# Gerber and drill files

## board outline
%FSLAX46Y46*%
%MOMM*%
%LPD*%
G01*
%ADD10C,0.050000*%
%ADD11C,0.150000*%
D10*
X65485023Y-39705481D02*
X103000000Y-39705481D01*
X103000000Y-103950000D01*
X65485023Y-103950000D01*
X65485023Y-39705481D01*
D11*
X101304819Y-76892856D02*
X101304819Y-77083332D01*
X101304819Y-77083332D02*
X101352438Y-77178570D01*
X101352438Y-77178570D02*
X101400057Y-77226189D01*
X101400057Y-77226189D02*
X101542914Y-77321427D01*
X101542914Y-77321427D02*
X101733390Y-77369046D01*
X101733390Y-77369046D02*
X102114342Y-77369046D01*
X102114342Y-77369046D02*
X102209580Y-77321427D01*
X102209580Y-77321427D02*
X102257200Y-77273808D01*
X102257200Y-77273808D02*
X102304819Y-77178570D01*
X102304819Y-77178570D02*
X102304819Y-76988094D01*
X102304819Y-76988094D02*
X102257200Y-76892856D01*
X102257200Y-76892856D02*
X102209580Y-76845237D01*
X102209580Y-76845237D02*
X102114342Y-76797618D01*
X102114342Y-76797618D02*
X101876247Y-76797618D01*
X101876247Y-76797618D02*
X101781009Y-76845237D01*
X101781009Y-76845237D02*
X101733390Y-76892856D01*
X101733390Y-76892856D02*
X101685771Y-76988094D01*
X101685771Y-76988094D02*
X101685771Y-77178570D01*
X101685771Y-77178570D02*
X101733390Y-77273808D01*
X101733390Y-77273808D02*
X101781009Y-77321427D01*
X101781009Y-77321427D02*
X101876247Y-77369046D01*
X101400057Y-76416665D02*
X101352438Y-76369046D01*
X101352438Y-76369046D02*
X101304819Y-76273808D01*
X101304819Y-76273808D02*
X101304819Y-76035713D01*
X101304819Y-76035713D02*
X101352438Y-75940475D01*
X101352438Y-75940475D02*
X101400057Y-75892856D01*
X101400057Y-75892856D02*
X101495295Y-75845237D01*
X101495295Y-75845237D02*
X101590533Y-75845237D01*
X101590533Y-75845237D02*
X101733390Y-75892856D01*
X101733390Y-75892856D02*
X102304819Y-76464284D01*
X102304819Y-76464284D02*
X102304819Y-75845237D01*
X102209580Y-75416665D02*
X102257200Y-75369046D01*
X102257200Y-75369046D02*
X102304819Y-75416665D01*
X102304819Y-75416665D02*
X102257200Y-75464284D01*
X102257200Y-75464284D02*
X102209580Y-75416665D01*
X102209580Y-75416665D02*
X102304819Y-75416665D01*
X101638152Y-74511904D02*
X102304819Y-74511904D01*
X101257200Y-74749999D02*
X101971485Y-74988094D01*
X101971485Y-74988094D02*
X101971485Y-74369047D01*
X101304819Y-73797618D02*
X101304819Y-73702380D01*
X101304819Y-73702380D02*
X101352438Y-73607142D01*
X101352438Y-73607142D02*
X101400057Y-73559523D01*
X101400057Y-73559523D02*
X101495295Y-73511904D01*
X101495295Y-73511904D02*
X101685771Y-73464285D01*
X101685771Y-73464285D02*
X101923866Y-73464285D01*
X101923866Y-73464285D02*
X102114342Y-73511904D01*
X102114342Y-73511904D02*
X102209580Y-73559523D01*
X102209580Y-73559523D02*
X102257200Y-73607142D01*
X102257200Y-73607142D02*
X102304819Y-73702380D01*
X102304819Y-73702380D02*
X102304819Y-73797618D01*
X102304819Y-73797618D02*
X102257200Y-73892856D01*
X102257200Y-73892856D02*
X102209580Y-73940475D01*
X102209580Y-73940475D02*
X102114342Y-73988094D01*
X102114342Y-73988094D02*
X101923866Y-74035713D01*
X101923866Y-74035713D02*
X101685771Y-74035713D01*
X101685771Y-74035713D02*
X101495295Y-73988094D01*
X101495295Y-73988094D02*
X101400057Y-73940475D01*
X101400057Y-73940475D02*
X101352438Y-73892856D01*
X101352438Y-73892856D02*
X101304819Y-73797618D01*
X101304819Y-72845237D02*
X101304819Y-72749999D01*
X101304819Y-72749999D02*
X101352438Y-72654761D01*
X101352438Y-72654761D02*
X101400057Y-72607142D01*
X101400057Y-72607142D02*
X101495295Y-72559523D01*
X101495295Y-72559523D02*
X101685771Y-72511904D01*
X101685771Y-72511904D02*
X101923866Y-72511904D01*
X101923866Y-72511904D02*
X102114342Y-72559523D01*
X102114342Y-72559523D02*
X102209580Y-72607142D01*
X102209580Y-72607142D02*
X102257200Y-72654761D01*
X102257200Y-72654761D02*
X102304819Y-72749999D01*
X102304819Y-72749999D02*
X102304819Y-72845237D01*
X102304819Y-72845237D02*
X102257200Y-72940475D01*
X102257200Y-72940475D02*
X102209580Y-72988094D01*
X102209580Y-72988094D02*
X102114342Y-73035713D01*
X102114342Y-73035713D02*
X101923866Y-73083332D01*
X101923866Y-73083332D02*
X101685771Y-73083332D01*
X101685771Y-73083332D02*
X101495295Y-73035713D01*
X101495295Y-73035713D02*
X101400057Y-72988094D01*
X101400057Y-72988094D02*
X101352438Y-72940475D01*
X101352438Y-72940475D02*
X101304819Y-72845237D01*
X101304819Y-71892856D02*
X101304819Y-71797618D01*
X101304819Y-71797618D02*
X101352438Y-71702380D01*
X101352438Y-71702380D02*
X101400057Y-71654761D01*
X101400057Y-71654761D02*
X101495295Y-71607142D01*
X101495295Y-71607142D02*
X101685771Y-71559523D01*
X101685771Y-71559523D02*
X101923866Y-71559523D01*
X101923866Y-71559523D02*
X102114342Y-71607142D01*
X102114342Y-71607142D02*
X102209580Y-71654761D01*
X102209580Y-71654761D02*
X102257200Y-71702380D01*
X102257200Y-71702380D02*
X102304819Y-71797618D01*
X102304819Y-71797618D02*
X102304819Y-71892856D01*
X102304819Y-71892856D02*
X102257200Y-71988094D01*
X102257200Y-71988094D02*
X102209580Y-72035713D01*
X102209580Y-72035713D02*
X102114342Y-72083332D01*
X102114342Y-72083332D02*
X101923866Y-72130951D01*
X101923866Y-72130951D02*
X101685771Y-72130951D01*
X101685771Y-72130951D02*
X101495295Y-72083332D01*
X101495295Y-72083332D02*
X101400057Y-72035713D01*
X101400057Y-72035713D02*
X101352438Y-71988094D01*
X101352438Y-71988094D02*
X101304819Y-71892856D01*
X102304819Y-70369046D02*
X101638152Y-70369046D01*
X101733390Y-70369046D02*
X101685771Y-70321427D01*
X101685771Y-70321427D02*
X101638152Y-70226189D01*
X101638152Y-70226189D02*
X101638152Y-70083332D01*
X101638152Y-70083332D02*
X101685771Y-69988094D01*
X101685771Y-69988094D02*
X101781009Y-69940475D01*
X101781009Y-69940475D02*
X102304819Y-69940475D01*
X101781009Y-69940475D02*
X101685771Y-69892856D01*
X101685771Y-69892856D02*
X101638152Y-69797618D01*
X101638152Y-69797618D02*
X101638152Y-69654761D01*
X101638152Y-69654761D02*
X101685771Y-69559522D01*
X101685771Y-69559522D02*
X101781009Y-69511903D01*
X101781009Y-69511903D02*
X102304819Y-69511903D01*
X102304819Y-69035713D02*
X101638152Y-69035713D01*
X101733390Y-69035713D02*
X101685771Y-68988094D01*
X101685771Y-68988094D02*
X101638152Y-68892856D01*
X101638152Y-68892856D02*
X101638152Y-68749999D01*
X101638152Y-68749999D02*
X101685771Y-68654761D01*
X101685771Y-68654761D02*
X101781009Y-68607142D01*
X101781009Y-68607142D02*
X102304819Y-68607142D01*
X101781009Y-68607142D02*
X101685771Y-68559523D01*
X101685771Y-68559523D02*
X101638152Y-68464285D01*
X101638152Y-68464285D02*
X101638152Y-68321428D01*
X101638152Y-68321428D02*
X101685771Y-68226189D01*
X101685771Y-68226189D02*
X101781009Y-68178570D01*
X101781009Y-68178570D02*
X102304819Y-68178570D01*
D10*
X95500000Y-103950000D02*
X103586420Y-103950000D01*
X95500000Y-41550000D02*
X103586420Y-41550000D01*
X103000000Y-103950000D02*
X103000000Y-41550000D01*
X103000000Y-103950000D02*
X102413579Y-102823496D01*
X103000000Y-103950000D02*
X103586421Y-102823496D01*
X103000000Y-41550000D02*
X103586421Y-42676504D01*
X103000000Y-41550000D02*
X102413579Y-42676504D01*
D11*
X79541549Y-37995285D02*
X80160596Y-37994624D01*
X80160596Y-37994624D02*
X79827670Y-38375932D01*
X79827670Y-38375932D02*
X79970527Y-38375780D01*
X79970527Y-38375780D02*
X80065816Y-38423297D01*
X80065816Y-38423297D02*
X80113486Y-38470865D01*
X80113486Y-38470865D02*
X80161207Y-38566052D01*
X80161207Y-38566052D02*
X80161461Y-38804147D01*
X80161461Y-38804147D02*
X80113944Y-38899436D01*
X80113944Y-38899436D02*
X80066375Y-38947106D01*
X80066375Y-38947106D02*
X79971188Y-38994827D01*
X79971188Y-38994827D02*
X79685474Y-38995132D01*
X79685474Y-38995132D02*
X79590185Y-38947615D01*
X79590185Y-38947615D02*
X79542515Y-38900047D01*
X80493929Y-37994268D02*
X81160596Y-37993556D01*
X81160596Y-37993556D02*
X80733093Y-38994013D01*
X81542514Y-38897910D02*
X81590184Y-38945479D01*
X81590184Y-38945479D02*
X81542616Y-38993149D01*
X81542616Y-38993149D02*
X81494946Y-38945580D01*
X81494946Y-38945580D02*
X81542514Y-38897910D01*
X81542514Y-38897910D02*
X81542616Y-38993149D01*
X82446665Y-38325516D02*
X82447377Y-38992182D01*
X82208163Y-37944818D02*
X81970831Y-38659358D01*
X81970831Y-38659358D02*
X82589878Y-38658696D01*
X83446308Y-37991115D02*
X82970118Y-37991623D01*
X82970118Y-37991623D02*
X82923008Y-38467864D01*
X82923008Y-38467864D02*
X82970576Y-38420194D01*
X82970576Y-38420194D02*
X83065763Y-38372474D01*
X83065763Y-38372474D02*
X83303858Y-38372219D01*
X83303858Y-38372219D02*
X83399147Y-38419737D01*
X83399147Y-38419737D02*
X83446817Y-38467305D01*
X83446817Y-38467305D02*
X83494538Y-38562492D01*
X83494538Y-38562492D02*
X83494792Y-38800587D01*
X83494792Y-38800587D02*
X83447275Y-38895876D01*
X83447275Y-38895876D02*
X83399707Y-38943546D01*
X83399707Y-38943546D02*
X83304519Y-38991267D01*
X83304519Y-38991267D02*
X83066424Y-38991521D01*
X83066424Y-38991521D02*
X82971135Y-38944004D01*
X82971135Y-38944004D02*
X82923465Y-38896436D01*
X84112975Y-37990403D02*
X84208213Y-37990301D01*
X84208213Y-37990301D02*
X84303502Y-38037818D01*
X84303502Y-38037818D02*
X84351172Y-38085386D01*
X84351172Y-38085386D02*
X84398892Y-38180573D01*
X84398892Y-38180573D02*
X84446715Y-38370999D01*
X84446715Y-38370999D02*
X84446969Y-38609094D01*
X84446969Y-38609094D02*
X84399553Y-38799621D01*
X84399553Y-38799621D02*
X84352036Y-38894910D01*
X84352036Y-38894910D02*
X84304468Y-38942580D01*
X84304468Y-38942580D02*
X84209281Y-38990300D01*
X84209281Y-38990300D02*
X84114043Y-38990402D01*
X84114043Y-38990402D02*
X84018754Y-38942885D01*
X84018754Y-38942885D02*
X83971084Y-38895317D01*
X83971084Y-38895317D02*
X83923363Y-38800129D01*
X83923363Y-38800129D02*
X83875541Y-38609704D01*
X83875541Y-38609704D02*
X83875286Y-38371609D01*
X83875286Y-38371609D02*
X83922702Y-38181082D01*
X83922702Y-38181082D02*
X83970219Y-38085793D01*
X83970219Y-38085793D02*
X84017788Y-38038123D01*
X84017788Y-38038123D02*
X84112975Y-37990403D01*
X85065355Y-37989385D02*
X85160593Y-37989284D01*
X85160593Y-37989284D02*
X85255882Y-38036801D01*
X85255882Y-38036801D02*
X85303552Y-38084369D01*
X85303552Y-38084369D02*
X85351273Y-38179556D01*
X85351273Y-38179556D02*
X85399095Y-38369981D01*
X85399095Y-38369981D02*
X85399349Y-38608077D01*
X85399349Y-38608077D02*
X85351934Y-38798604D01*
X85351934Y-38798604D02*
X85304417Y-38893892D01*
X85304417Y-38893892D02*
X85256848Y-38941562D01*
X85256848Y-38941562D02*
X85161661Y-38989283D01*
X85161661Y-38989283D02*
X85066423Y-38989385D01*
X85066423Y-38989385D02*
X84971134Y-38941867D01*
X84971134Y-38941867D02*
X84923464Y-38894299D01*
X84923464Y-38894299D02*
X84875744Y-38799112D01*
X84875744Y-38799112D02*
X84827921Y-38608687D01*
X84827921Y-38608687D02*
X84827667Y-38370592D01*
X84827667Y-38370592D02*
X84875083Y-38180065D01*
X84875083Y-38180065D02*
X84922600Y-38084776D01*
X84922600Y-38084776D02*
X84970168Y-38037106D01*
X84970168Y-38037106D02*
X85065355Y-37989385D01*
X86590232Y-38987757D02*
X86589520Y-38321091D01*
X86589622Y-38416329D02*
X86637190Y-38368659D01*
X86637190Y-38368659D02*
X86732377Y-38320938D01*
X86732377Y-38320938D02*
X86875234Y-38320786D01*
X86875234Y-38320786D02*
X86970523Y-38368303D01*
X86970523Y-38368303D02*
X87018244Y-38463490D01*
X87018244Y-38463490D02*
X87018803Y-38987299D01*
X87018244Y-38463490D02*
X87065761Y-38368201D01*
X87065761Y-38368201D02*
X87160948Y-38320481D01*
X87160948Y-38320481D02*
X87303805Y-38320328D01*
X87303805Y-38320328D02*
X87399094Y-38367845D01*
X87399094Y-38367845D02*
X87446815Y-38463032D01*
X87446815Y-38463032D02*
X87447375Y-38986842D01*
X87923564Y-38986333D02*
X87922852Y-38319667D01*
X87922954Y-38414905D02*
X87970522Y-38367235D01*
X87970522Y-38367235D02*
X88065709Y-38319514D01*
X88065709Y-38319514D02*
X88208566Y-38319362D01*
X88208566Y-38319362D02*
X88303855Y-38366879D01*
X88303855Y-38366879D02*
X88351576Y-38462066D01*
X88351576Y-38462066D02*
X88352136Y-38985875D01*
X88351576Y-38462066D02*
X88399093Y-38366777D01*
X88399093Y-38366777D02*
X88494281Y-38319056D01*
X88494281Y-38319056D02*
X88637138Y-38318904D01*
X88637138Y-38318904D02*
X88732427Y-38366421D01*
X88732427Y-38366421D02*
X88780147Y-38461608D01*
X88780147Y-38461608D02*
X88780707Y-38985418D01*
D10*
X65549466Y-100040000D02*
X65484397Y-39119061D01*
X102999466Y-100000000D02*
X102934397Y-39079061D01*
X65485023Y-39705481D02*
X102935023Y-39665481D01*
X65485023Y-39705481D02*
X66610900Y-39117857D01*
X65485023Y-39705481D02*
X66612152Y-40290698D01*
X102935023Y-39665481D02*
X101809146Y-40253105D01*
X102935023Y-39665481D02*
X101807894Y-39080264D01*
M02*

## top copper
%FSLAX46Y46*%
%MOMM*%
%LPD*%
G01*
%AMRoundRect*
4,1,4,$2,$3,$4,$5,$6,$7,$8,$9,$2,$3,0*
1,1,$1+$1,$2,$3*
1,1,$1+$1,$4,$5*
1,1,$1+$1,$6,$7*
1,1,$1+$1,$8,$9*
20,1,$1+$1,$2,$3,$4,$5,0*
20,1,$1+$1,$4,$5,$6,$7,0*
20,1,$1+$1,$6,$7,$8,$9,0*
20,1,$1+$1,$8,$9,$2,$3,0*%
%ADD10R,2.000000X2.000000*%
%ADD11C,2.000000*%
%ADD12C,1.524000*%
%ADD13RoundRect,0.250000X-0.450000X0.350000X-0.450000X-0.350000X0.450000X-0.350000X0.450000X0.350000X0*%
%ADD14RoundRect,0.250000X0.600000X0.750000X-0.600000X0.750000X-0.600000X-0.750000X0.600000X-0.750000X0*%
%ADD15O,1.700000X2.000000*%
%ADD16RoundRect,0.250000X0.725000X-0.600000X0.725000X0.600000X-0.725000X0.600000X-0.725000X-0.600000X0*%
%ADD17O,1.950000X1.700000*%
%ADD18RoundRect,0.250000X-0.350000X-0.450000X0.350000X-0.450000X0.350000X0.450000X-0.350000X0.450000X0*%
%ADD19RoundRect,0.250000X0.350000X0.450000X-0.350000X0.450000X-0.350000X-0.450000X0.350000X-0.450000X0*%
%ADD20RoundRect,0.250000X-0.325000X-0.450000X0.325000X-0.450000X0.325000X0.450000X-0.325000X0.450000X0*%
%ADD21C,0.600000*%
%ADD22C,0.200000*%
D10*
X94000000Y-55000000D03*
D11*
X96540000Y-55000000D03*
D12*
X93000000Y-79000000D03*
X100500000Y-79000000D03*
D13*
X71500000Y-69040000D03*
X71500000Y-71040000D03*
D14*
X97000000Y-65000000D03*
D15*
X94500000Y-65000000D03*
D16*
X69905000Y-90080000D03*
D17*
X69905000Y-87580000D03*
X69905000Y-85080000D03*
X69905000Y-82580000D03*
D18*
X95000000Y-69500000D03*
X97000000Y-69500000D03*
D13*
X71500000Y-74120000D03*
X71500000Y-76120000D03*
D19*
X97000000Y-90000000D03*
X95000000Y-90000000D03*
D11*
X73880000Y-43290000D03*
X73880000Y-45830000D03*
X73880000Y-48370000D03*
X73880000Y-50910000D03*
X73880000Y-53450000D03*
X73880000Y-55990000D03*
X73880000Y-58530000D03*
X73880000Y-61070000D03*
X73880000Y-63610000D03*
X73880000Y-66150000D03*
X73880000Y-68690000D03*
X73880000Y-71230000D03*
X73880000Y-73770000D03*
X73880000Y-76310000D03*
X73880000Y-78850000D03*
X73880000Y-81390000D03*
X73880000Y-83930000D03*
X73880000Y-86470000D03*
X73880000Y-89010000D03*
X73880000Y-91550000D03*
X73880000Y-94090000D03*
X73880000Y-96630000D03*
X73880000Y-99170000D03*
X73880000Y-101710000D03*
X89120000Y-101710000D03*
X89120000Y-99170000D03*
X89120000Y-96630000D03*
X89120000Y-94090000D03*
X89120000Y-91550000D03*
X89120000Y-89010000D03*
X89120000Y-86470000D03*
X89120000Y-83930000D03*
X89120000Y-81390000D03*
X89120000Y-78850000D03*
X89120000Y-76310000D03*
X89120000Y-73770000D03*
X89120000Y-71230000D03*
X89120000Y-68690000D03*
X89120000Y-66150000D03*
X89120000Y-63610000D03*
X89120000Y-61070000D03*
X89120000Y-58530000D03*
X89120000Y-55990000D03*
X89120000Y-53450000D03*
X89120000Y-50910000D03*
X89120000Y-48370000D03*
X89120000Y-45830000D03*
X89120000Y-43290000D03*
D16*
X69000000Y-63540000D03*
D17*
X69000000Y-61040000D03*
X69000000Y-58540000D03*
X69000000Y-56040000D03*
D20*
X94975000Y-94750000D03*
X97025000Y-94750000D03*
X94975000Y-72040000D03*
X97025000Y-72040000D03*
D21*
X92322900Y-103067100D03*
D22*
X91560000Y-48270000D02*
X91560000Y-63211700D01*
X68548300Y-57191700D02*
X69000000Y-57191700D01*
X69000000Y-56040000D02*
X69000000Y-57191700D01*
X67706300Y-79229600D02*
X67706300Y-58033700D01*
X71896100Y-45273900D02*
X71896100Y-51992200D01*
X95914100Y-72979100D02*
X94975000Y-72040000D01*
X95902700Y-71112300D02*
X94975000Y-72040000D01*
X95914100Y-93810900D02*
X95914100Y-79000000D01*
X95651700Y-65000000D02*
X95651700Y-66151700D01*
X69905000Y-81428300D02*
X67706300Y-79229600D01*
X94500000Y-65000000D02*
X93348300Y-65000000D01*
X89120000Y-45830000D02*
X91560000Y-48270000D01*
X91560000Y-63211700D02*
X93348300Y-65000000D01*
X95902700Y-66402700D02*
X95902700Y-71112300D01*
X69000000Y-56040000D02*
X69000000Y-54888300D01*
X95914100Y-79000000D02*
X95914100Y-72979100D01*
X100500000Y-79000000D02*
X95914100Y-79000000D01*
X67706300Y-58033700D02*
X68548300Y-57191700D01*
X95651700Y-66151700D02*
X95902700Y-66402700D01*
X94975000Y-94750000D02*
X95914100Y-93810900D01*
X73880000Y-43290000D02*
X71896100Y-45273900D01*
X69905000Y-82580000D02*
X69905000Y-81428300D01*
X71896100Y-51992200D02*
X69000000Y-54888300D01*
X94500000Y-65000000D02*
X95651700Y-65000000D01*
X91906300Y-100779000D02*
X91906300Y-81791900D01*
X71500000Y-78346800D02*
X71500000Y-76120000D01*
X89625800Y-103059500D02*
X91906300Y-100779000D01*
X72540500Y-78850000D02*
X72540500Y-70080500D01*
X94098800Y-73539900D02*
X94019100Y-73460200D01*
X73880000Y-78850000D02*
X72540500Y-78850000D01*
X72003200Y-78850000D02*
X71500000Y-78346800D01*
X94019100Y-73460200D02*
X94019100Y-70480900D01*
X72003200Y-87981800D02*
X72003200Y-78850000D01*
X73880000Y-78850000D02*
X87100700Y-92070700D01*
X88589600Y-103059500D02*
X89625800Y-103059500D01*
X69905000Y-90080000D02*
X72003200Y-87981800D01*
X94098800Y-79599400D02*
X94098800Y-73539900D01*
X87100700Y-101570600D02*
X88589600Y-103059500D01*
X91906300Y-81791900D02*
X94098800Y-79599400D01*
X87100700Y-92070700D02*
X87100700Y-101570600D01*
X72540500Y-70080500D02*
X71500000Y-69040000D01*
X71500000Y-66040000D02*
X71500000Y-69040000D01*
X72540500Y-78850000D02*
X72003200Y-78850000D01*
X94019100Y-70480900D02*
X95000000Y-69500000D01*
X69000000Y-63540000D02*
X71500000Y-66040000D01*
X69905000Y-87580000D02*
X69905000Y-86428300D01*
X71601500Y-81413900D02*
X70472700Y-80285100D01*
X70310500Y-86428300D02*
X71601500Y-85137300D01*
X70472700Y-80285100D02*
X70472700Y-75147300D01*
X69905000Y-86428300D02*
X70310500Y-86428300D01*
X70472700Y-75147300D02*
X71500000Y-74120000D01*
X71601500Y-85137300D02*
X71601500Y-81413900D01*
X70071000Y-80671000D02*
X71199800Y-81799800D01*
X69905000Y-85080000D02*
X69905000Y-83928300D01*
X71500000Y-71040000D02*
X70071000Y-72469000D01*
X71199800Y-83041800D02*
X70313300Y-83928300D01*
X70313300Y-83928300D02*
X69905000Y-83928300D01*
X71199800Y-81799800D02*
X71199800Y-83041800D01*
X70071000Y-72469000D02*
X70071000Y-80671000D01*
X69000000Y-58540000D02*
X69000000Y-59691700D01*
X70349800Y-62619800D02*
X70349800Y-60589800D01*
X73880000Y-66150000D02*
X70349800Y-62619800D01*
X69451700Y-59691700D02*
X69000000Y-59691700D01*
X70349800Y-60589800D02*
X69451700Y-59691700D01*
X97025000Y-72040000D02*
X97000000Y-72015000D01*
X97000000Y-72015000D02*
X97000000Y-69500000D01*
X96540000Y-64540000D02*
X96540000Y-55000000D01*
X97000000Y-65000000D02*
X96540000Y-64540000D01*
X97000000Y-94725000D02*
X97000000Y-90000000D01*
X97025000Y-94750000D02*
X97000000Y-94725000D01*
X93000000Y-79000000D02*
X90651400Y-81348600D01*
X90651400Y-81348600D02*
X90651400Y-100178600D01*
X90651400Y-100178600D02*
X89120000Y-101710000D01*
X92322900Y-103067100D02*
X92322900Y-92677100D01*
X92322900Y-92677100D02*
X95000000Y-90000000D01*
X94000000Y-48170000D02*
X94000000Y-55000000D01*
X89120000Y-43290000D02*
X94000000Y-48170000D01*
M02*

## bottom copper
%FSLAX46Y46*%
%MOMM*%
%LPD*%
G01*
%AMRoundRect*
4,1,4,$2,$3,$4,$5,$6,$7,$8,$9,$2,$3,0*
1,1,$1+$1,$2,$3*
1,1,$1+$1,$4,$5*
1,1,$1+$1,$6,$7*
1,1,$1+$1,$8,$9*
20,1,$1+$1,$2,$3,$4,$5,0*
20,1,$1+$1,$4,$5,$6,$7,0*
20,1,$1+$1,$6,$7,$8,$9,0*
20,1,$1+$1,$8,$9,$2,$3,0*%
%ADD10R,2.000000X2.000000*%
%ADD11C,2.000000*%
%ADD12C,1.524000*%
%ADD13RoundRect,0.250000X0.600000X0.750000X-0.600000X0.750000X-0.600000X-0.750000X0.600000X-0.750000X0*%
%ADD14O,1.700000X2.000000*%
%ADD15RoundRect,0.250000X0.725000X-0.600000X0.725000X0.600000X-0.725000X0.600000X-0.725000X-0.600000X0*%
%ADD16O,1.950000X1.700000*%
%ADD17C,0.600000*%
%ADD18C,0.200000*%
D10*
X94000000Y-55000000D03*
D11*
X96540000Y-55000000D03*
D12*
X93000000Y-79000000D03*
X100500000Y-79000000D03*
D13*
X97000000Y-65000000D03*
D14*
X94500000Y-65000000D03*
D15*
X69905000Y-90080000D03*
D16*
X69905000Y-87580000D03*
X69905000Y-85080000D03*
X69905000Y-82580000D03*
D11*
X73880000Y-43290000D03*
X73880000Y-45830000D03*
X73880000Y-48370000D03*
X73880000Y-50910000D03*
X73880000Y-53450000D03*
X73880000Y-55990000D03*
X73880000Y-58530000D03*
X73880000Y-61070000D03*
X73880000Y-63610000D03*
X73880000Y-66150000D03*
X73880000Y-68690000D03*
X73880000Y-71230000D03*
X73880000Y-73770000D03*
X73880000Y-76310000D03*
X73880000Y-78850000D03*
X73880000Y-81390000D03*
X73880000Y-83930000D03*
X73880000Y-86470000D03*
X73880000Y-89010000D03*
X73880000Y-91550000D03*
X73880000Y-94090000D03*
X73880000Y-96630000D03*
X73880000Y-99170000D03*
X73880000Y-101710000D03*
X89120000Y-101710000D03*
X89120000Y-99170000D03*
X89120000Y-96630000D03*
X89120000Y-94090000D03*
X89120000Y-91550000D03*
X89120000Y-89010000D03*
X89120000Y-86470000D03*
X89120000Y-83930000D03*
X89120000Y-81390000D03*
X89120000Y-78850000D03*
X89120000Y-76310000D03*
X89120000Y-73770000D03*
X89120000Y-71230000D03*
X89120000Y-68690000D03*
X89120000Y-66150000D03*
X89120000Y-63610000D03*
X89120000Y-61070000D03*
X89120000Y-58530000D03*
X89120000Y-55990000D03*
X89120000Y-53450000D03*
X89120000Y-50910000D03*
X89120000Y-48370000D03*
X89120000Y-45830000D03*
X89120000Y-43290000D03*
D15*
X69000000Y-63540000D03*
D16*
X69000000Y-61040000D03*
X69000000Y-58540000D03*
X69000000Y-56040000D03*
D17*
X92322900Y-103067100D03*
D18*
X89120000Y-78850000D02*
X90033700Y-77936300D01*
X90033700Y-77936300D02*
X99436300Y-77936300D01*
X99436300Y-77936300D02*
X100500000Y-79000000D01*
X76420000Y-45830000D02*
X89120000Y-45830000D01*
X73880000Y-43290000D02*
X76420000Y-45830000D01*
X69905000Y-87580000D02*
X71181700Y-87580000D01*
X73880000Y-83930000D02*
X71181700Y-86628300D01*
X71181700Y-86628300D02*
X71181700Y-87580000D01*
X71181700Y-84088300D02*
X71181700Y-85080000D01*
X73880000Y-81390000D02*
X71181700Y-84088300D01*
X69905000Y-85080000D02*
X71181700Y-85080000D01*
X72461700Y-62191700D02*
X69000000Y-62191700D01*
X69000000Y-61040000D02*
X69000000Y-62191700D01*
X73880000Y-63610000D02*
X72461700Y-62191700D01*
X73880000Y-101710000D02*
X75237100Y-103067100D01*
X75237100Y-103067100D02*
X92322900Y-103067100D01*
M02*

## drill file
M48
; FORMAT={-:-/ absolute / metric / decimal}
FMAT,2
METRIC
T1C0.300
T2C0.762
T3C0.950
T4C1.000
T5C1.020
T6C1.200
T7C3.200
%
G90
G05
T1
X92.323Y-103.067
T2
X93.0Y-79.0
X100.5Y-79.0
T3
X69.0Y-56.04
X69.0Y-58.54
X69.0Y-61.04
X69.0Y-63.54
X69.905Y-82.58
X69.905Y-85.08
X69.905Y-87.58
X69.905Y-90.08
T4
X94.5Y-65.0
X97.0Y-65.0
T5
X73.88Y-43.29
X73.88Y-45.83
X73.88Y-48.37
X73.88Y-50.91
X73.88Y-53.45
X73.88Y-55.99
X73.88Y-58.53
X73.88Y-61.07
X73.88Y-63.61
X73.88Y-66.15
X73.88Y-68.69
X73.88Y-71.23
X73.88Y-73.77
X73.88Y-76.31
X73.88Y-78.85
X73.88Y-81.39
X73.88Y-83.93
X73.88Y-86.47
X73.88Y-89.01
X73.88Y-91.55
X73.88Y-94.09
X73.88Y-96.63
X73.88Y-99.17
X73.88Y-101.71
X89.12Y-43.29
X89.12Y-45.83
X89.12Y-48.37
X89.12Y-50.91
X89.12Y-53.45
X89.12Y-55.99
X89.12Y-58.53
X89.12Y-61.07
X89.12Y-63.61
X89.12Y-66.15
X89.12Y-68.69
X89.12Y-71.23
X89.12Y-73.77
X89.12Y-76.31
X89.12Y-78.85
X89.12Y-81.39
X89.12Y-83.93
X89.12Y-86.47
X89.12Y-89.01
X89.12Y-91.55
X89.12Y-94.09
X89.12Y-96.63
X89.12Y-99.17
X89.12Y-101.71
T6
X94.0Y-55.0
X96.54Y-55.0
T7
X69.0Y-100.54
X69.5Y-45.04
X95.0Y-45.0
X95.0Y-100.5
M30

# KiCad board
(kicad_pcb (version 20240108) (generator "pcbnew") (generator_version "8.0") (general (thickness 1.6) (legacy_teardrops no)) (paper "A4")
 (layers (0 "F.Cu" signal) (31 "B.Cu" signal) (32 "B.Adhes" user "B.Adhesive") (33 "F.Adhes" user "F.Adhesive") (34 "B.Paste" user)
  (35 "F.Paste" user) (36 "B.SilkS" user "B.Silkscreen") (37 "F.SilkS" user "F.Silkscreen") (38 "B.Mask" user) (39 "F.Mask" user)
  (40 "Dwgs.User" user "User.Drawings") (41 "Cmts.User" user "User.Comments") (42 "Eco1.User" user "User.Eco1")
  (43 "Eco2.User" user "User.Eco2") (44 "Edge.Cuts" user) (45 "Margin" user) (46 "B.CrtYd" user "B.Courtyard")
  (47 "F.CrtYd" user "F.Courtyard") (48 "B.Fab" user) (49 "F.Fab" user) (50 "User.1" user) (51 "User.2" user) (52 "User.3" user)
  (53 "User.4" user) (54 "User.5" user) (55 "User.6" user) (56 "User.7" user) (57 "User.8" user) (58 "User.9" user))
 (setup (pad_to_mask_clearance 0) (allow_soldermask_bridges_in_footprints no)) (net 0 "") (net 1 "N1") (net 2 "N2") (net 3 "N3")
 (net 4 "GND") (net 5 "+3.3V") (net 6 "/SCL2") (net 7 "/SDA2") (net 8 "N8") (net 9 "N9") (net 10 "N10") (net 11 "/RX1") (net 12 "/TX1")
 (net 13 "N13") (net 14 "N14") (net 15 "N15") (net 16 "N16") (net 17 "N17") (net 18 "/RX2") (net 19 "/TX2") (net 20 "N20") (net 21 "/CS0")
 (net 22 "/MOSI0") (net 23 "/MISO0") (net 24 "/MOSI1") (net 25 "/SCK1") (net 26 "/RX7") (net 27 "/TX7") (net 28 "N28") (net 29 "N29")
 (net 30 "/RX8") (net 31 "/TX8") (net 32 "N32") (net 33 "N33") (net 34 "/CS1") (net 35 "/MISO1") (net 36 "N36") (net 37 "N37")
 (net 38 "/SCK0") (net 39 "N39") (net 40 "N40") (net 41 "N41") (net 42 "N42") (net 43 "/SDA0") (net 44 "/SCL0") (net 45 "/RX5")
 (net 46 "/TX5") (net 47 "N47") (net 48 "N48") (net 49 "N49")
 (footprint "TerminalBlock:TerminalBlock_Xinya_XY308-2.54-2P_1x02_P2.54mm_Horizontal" (layer "F.Cu") (at 94 55)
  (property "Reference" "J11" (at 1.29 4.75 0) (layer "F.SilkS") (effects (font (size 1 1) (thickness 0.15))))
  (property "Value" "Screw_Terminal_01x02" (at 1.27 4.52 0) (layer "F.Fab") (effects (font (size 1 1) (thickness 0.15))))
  (pad "1" thru_hole rect (at 0 0) (size 2 2) (drill 1.2) (layers "*.Cu" "*.Mask") (remove_unused_layers no) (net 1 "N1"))
  (pad "2" thru_hole circle (at 2.54 0) (size 2 2) (drill 1.2) (layers "*.Cu" "*.Mask") (remove_unused_layers no) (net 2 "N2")))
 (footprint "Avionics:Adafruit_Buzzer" (layer "F.Cu") (at 97 79)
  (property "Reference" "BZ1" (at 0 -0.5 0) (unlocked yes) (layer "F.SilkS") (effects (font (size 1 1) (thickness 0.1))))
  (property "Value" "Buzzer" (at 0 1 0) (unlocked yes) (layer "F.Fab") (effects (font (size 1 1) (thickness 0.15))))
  (pad "1" thru_hole circle (at -4 0) (size 1.524 1.524) (drill 0.762) (layers "*.Cu" "*.Mask") (remove_unused_layers no) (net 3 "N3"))
  (pad "2" thru_hole circle (at 3.5 0) (size 1.524 1.524) (drill 0.762) (layers "*.Cu" "*.Mask") (remove_unused_layers no) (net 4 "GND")))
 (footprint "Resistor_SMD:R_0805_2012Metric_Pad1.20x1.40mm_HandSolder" (layer "F.Cu") (at 71.5 70.04 -90)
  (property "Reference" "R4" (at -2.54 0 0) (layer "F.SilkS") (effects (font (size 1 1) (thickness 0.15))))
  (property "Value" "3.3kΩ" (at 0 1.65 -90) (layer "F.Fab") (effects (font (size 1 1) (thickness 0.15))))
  (pad "1" smd roundrect (at -1 0 270) (size 1.2 1.4) (layers "F.Cu" "F.Paste" "F.Mask") (roundrect_rratio 0.208333) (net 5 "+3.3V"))
  (pad "2" smd roundrect (at 1 0 270) (size 1.2 1.4) (layers "F.Cu" "F.Paste" "F.Mask") (roundrect_rratio 0.208333) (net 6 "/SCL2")))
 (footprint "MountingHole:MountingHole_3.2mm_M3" (layer "F.Cu") (at 95 45)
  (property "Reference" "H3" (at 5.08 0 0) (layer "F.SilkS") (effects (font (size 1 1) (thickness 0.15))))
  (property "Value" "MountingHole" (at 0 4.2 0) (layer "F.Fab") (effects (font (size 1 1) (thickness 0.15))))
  (pad "" np_thru_hole circle (at 0 0) (size 3.2 3.2) (drill 3.2) (layers "*.Cu" "*.Mask")))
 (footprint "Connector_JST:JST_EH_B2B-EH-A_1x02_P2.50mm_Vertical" (layer "F.Cu") (at 97 65 180)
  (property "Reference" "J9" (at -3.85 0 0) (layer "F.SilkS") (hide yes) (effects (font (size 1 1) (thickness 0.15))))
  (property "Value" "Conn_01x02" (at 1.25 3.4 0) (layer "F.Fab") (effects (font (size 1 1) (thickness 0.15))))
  (pad "1" thru_hole roundrect (at 0 0 180) (size 1.7 2) (drill 1) (layers "*.Cu" "*.Mask") (remove_unused_layers no)
   (roundrect_rratio 0.147059) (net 2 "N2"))
  (pad "2" thru_hole oval (at 2.5 0 180) (size 1.7 2) (drill 1) (layers "*.Cu" "*.Mask") (remove_unused_layers no) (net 4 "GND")))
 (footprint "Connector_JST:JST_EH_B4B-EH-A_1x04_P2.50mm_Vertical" (layer "F.Cu") (at 69.905 90.08 90)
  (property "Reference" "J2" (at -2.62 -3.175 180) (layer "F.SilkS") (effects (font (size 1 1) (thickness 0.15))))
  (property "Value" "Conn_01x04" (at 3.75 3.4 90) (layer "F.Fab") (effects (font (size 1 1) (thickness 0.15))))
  (pad "1" thru_hole roundrect (at 0 0 90) (size 1.7 1.95) (drill 0.95) (layers "*.Cu" "*.Mask") (remove_unused_layers no)
   (roundrect_rratio 0.147059) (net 5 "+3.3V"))
  (pad "2" thru_hole oval (at 2.5 0 90) (size 1.7 1.95) (drill 0.95) (layers "*.Cu" "*.Mask") (remove_unused_layers no) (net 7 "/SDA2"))
  (pad "3" thru_hole oval (at 5 0 90) (size 1.7 1.95) (drill 0.95) (layers "*.Cu" "*.Mask") (remove_unused_layers no) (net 6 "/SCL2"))
  (pad "4" thru_hole oval (at 7.5 0 90) (size 1.7 1.95) (drill 0.95) (layers "*.Cu" "*.Mask") (remove_unused_layers no) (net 4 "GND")))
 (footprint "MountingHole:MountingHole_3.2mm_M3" (layer "F.Cu") (at 69.5 45.04)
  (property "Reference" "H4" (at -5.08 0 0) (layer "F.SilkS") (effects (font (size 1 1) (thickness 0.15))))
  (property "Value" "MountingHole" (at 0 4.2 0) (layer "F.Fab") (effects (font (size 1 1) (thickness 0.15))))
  (pad "" np_thru_hole circle (at 0 0) (size 3.2 3.2) (drill 3.2) (layers "*.Cu" "*.Mask")))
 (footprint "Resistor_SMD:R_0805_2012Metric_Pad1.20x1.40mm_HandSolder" (layer "F.Cu") (at 96 69.5)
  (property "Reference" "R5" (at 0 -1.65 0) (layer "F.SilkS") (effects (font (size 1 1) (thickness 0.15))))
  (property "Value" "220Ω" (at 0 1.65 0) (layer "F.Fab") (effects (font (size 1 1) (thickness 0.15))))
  (pad "1" smd roundrect (at -1 0) (size 1.2 1.4) (layers "F.Cu" "F.Paste" "F.Mask") (roundrect_rratio 0.208333) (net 5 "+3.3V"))
  (pad "2" smd roundrect (at 1 0) (size 1.2 1.4) (layers "F.Cu" "F.Paste" "F.Mask") (roundrect_rratio 0.208333) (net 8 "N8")))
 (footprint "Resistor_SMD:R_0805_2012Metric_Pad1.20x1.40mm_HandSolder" (layer "F.Cu") (at 71.5 75.12 -90)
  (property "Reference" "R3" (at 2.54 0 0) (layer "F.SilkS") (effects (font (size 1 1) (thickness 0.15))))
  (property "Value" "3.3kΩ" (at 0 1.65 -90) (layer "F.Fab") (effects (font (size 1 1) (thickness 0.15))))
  (pad "1" smd roundrect (at -1 0 270) (size 1.2 1.4) (layers "F.Cu" "F.Paste" "F.Mask") (roundrect_rratio 0.208333) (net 7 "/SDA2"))
  (pad "2" smd roundrect (at 1 0 270) (size 1.2 1.4) (layers "F.Cu" "F.Paste" "F.Mask") (roundrect_rratio 0.208333) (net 5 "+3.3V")))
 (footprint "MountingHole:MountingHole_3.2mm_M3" (layer "F.Cu") (at 69 100.54)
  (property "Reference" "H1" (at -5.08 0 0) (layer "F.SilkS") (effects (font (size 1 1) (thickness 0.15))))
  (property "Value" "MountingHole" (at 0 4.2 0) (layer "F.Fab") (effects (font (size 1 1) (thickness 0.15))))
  (pad "" np_thru_hole circle (at 0 0) (size 3.2 3.2) (drill 3.2) (layers "*.Cu" "*.Mask")))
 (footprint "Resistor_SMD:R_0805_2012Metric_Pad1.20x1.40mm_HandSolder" (layer "F.Cu") (at 96 90 180)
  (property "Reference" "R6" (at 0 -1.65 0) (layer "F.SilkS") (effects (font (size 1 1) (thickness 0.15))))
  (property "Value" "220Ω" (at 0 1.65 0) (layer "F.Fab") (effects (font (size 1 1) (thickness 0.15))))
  (pad "1" smd roundrect (at -1 0 180) (size 1.2 1.4) (layers "F.Cu" "F.Paste" "F.Mask") (roundrect_rratio 0.208333) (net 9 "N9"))
  (pad "2" smd roundrect (at 1 0 180) (size 1.2 1.4) (layers "F.Cu" "F.Paste" "F.Mask") (roundrect_rratio 0.208333) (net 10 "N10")))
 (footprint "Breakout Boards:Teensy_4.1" (layer "F.Cu") (at 81.5 72.5)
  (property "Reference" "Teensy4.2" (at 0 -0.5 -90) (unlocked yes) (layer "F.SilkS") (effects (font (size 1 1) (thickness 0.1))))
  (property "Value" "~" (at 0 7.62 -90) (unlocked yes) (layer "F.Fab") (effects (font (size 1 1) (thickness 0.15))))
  (pad "0" thru_hole circle (at -7.62 -29.21) (size 2 2) (drill 1.02) (layers "*.Cu" "*.Mask") (remove_unused_layers no) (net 4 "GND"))
  (pad "1" thru_hole circle (at -7.62 -26.67) (size 2 2) (drill 1.02) (layers "*.Cu" "*.Mask") (remove_unused_layers no) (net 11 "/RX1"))
  (pad "2" thru_hole circle (at -7.62 -24.13) (size 2 2) (drill 1.02) (layers "*.Cu" "*.Mask") (remove_unused_layers no) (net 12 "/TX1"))
  (pad "3" thru_hole circle (at -7.62 -21.59) (size 2 2) (drill 1.02) (layers "*.Cu" "*.Mask") (remove_unused_layers no) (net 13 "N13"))
  (pad "4" thru_hole circle (at -7.62 -19.05) (size 2 2) (drill 1.02) (layers "*.Cu" "*.Mask") (remove_unused_layers no) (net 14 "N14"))
  (pad "5" thru_hole circle (at -7.62 -16.51) (size 2 2) (drill 1.02) (layers "*.Cu" "*.Mask") (remove_unused_layers no) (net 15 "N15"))
  (pad "6" thru_hole circle (at -7.62 -13.97) (size 2 2) (drill 1.02) (layers "*.Cu" "*.Mask") (remove_unused_layers no) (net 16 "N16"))
  (pad "7" thru_hole circle (at -7.62 -11.43) (size 2 2) (drill 1.02) (layers "*.Cu" "*.Mask") (remove_unused_layers no) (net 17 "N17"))
  (pad "8" thru_hole circle (at -7.62 -8.89) (size 2 2) (drill 1.02) (layers "*.Cu" "*.Mask") (remove_unused_layers no) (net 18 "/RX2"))
  (pad "9" thru_hole circle (at -7.62 -6.35) (size 2 2) (drill 1.02) (layers "*.Cu" "*.Mask") (remove_unused_layers no) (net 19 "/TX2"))
  (pad "10" thru_hole circle (at -7.62 -3.81) (size 2 2) (drill 1.02) (layers "*.Cu" "*.Mask") (remove_unused_layers no) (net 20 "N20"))
  (pad "11" thru_hole circle (at -7.62 -1.27) (size 2 2) (drill 1.02) (layers "*.Cu" "*.Mask") (remove_unused_layers no) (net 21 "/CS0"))
  (pad "12" thru_hole circle (at -7.62 1.27) (size 2 2) (drill 1.02) (layers "*.Cu" "*.Mask") (remove_unused_layers no) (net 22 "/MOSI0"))
  (pad "13" thru_hole circle (at -7.62 3.81) (size 2 2) (drill 1.02) (layers "*.Cu" "*.Mask") (remove_unused_layers no) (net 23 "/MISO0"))
  (pad "14" thru_hole circle (at -7.62 6.35) (size 2 2) (drill 1.02) (layers "*.Cu" "*.Mask") (remove_unused_layers no) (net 5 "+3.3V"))
  (pad "15" thru_hole circle (at -7.62 8.89) (size 2 2) (drill 1.02) (layers "*.Cu" "*.Mask") (remove_unused_layers no) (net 6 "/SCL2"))
  (pad "16" thru_hole circle (at -7.62 11.43) (size 2 2) (drill 1.02) (layers "*.Cu" "*.Mask") (remove_unused_layers no) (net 7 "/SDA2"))
  (pad "17" thru_hole circle (at -7.62 13.97) (size 2 2) (drill 1.02) (layers "*.Cu" "*.Mask") (remove_unused_layers no) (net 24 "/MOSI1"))
  (pad "18" thru_hole circle (at -7.62 16.51) (size 2 2) (drill 1.02) (layers "*.Cu" "*.Mask") (remove_unused_layers no) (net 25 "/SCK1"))
  (pad "19" thru_hole circle (at -7.62 19.05) (size 2 2) (drill 1.02) (layers "*.Cu" "*.Mask") (remove_unused_layers no) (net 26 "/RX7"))
  (pad "20" thru_hole circle (at -7.62 21.59) (size 2 2) (drill 1.02) (layers "*.Cu" "*.Mask") (remove_unused_layers no) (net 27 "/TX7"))
  (pad "21" thru_hole circle (at -7.62 24.13) (size 2 2) (drill 1.02) (layers "*.Cu" "*.Mask") (remove_unused_layers no) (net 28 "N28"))
  (pad "22" thru_hole circle (at -7.62 26.67) (size 2 2) (drill 1.02) (layers "*.Cu" "*.Mask") (remove_unused_layers no) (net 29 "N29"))
  (pad "23" thru_hole circle (at -7.62 29.21) (size 2 2) (drill 1.02) (layers "*.Cu" "*.Mask") (remove_unused_layers no) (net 10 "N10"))
  (pad "24" thru_hole circle (at 7.62 29.21) (size 2 2) (drill 1.02) (layers "*.Cu" "*.Mask") (remove_unused_layers no) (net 3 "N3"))
  (pad "25" thru_hole circle (at 7.62 26.67) (size 2 2) (drill 1.02) (layers "*.Cu" "*.Mask") (remove_unused_layers no) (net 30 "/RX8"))
  (pad "26" thru_hole circle (at 7.62 24.13) (size 2 2) (drill 1.02) (layers "*.Cu" "*.Mask") (remove_unused_layers no) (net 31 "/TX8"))
  (pad "27" thru_hole circle (at 7.62 21.59) (size 2 2) (drill 1.02) (layers "*.Cu" "*.Mask") (remove_unused_layers no) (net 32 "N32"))
  (pad "28" thru_hole circle (at 7.62 19.05) (size 2 2) (drill 1.02) (layers "*.Cu" "*.Mask") (remove_unused_layers no) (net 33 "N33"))
  (pad "29" thru_hole circle (at 7.62 16.51) (size 2 2) (drill 1.02) (layers "*.Cu" "*.Mask") (remove_unused_layers no) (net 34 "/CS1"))
  (pad "30" thru_hole circle (at 7.62 13.97) (size 2 2) (drill 1.02) (layers "*.Cu" "*.Mask") (remove_unused_layers no) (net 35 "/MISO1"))
  (pad "31" thru_hole circle (at 7.62 11.43) (size 2 2) (drill 1.02) (layers "*.Cu" "*.Mask") (remove_unused_layers no) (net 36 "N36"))
  (pad "32" thru_hole circle (at 7.62 8.89) (size 2 2) (drill 1.02) (layers "*.Cu" "*.Mask") (remove_unused_layers no) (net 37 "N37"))
  (pad "33" thru_hole circle (at 7.62 6.35) (size 2 2) (drill 1.02) (layers "*.Cu" "*.Mask") (remove_unused_layers no) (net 4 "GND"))
  (pad "34" thru_hole circle (at 7.62 3.81) (size 2 2) (drill 1.02) (layers "*.Cu" "*.Mask") (remove_unused_layers no) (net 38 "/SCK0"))
  (pad "35" thru_hole circle (at 7.62 1.27) (size 2 2) (drill 1.02) (layers "*.Cu" "*.Mask") (remove_unused_layers no) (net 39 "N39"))
  (pad "36" thru_hole circle (at 7.62 -1.27) (size 2 2) (drill 1.02) (layers "*.Cu" "*.Mask") (remove_unused_layers no) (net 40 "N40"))
  (pad "37" thru_hole circle (at 7.62 -3.81) (size 2 2) (drill 1.02) (layers "*.Cu" "*.Mask") (remove_unused_layers no) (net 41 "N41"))
  (pad "38" thru_hole circle (at 7.62 -6.35) (size 2 2) (drill 1.02) (layers "*.Cu" "*.Mask") (remove_unused_layers no) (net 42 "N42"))
  (pad "39" thru_hole circle (at 7.62 -8.89) (size 2 2) (drill 1.02) (layers "*.Cu" "*.Mask") (remove_unused_layers no) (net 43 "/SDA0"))
  (pad "40" thru_hole circle (at 7.62 -11.43) (size 2 2) (drill 1.02) (layers "*.Cu" "*.Mask") (remove_unused_layers no) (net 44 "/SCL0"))
  (pad "41" thru_hole circle (at 7.62 -13.97) (size 2 2) (drill 1.02) (layers "*.Cu" "*.Mask") (remove_unused_layers no) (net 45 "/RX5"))
  (pad "42" thru_hole circle (at 7.62 -16.51) (size 2 2) (drill 1.02) (layers "*.Cu" "*.Mask") (remove_unused_layers no) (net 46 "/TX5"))
  (pad "43" thru_hole circle (at 7.62 -19.05) (size 2 2) (drill 1.02) (layers "*.Cu" "*.Mask") (remove_unused_layers no) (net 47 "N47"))
  (pad "44" thru_hole circle (at 7.62 -21.59) (size 2 2) (drill 1.02) (layers "*.Cu" "*.Mask") (remove_unused_layers no) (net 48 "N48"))
  (pad "45" thru_hole circle (at 7.62 -24.13) (size 2 2) (drill 1.02) (layers "*.Cu" "*.Mask") (remove_unused_layers no) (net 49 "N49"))
  (pad "46" thru_hole circle (at 7.62 -26.67) (size 2 2) (drill 1.02) (layers "*.Cu" "*.Mask") (remove_unused_layers no) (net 4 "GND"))
  (pad "47" thru_hole circle (at 7.62 -29.21) (size 2 2) (drill 1.02) (layers "*.Cu" "*.Mask") (remove_unused_layers no) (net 1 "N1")))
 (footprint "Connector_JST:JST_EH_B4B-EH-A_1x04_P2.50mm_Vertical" (layer "F.Cu") (at 69 63.54 90)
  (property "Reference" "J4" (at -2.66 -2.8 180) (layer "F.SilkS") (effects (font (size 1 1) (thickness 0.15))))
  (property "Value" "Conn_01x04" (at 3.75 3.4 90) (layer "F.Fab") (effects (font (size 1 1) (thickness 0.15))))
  (pad "1" thru_hole roundrect (at 0 0 90) (size 1.7 1.95) (drill 0.95) (layers "*.Cu" "*.Mask") (remove_unused_layers no)
   (roundrect_rratio 0.147059) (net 5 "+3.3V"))
  (pad "2" thru_hole oval (at 2.5 0 90) (size 1.7 1.95) (drill 0.95) (layers "*.Cu" "*.Mask") (remove_unused_layers no) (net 18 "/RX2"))
  (pad "3" thru_hole oval (at 5 0 90) (size 1.7 1.95) (drill 0.95) (layers "*.Cu" "*.Mask") (remove_unused_layers no) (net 19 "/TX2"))
  (pad "4" thru_hole oval (at 7.5 0 90) (size 1.7 1.95) (drill 0.95) (layers "*.Cu" "*.Mask") (remove_unused_layers no) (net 4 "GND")))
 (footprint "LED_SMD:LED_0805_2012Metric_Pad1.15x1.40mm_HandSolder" (layer "F.Cu") (at 96 94.75)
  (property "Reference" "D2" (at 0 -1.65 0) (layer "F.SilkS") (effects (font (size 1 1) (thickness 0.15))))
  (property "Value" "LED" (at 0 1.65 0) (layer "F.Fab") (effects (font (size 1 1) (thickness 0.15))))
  (pad "1" smd roundrect (at -1.025 0) (size 1.15 1.4) (layers "F.Cu" "F.Paste" "F.Mask") (roundrect_rratio 0.217391) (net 4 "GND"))
  (pad "2" smd roundrect (at 1.025 0) (size 1.15 1.4) (layers "F.Cu" "F.Paste" "F.Mask") (roundrect_rratio 0.217391) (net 9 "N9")))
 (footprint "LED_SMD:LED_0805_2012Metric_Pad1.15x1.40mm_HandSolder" (layer "F.Cu") (at 96 72.04)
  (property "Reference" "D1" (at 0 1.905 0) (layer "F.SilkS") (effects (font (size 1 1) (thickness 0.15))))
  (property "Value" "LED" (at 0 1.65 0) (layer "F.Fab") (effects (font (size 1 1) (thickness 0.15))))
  (pad "1" smd roundrect (at -1.025 0) (size 1.15 1.4) (layers "F.Cu" "F.Paste" "F.Mask") (roundrect_rratio 0.217391) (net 4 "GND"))
  (pad "2" smd roundrect (at 1.025 0) (size 1.15 1.4) (layers "F.Cu" "F.Paste" "F.Mask") (roundrect_rratio 0.217391) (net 8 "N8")))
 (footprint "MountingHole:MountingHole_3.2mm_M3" (layer "F.Cu") (at 95 100.5)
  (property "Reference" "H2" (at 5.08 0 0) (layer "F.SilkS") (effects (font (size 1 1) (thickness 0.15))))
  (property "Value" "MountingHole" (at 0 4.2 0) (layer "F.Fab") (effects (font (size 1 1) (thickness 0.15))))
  (pad "" np_thru_hole circle (at 0 0) (size 3.2 3.2) (drill 3.2) (layers "*.Cu" "*.Mask")))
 (gr_rect (start 65.485023 39.705481) (end 103 103.95) (locked yes) (stroke (width 0.05) (type default)) (fill none) (layer "Edge.Cuts"))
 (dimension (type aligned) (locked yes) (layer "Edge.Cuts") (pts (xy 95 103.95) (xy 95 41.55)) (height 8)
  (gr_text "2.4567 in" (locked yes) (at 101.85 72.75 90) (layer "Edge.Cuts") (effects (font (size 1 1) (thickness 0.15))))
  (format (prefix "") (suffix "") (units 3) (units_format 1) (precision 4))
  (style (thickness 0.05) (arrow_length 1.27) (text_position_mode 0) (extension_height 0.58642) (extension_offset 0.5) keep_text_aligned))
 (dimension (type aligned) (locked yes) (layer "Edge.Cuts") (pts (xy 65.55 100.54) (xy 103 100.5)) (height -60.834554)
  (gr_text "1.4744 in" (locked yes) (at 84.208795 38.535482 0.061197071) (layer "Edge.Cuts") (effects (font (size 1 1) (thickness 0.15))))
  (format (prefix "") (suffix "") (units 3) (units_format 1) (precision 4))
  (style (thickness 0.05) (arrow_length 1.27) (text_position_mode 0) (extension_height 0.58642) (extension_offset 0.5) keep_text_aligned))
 (segment (start 91.56 48.27) (end 91.56 63.2117) (width 0.2) (layer "F.Cu") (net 4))
 (segment (start 68.5483 57.1917) (end 69 57.1917) (width 0.2) (layer "F.Cu") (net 4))
 (segment (start 69 56.04) (end 69 57.1917) (width 0.2) (layer "F.Cu") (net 4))
 (segment (start 67.7063 79.2296) (end 67.7063 58.0337) (width 0.2) (layer "F.Cu") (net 4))
 (segment (start 71.8961 45.2739) (end 71.8961 51.9922) (width 0.2) (layer "F.Cu") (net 4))
 (segment (start 95.9141 72.9791) (end 94.975 72.04) (width 0.2) (layer "F.Cu") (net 4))
 (segment (start 95.9027 71.1123) (end 94.975 72.04) (width 0.2) (layer "F.Cu") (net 4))
 (segment (start 95.9141 93.8109) (end 95.9141 79) (width 0.2) (layer "F.Cu") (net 4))
 (segment (start 95.6517 65) (end 95.6517 66.1517) (width 0.2) (layer "F.Cu") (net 4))
 (segment (start 69.905 81.4283) (end 67.7063 79.2296) (width 0.2) (layer "F.Cu") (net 4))
 (segment (start 94.5 65) (end 93.3483 65) (width 0.2) (layer "F.Cu") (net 4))
 (segment (start 89.12 45.83) (end 91.56 48.27) (width 0.2) (layer "F.Cu") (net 4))
 (segment (start 91.56 63.2117) (end 93.3483 65) (width 0.2) (layer "F.Cu") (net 4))
 (segment (start 95.9027 66.4027) (end 95.9027 71.1123) (width 0.2) (layer "F.Cu") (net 4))
 (segment (start 69 56.04) (end 69 54.8883) (width 0.2) (layer "F.Cu") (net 4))
 (segment (start 95.9141 79) (end 95.9141 72.9791) (width 0.2) (layer "F.Cu") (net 4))
 (segment (start 100.5 79) (end 95.9141 79) (width 0.2) (layer "F.Cu") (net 4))
 (segment (start 67.7063 58.0337) (end 68.5483 57.1917) (width 0.2) (layer "F.Cu") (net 4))
 (segment (start 95.6517 66.1517) (end 95.9027 66.4027) (width 0.2) (layer "F.Cu") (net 4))
 (segment (start 94.975 94.75) (end 95.9141 93.8109) (width 0.2) (layer "F.Cu") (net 4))
 (segment (start 73.88 43.29) (end 71.8961 45.2739) (width 0.2) (layer "F.Cu") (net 4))
 (segment (start 69.905 82.58) (end 69.905 81.4283) (width 0.2) (layer "F.Cu") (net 4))
 (segment (start 71.8961 51.9922) (end 69 54.8883) (width 0.2) (layer "F.Cu") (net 4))
 (segment (start 94.5 65) (end 95.6517 65) (width 0.2) (layer "F.Cu") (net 4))
 (segment (start 89.12 78.85) (end 90.0337 77.9363) (width 0.2) (layer "B.Cu") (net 4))
 (segment (start 90.0337 77.9363) (end 99.4363 77.9363) (width 0.2) (layer "B.Cu") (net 4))
 (segment (start 99.4363 77.9363) (end 100.5 79) (width 0.2) (layer "B.Cu") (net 4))
 (segment (start 76.42 45.83) (end 89.12 45.83) (width 0.2) (layer "B.Cu") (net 4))
 (segment (start 73.88 43.29) (end 76.42 45.83) (width 0.2) (layer "B.Cu") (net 4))
 (segment (start 91.9063 100.779) (end 91.9063 81.7919) (width 0.2) (layer "F.Cu") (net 5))
 (segment (start 71.5 78.3468) (end 71.5 76.12) (width 0.2) (layer "F.Cu") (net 5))
 (segment (start 89.6258 103.0595) (end 91.9063 100.779) (width 0.2) (layer "F.Cu") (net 5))
 (segment (start 72.5405 78.85) (end 72.5405 70.0805) (width 0.2) (layer "F.Cu") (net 5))
 (segment (start 94.0988 73.5399) (end 94.0191 73.4602) (width 0.2) (layer "F.Cu") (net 5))
 (segment (start 73.88 78.85) (end 72.5405 78.85) (width 0.2) (layer "F.Cu") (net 5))
 (segment (start 72.0032 78.85) (end 71.5 78.3468) (width 0.2) (layer "F.Cu") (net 5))
 (segment (start 94.0191 73.4602) (end 94.0191 70.4809) (width 0.2) (layer "F.Cu") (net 5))
 (segment (start 72.0032 87.9818) (end 72.0032 78.85) (width 0.2) (layer "F.Cu") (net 5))
 (segment (start 73.88 78.85) (end 87.1007 92.0707) (width 0.2) (layer "F.Cu") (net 5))
 (segment (start 88.5896 103.0595) (end 89.6258 103.0595) (width 0.2) (layer "F.Cu") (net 5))
 (segment (start 69.905 90.08) (end 72.0032 87.9818) (width 0.2) (layer "F.Cu") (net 5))
 (segment (start 94.0988 79.5994) (end 94.0988 73.5399) (width 0.2) (layer "F.Cu") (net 5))
 (segment (start 87.1007 101.5706) (end 88.5896 103.0595) (width 0.2) (layer "F.Cu") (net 5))
 (segment (start 91.9063 81.7919) (end 94.0988 79.5994) (width 0.2) (layer "F.Cu") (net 5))
 (segment (start 87.1007 92.0707) (end 87.1007 101.5706) (width 0.2) (layer "F.Cu") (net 5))
 (segment (start 72.5405 70.0805) (end 71.5 69.04) (width 0.2) (layer "F.Cu") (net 5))
 (segment (start 71.5 66.04) (end 71.5 69.04) (width 0.2) (layer "F.Cu") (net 5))
 (segment (start 72.5405 78.85) (end 72.0032 78.85) (width 0.2) (layer "F.Cu") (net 5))
 (segment (start 94.0191 70.4809) (end 95 69.5) (width 0.2) (layer "F.Cu") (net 5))
 (segment (start 69 63.54) (end 71.5 66.04) (width 0.2) (layer "F.Cu") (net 5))
 (segment (start 69.905 87.58) (end 69.905 86.4283) (width 0.2) (layer "F.Cu") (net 7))
 (segment (start 71.6015 81.4139) (end 70.4727 80.2851) (width 0.2) (layer "F.Cu") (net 7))
 (segment (start 70.3105 86.4283) (end 71.6015 85.1373) (width 0.2) (layer "F.Cu") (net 7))
 (segment (start 70.4727 80.2851) (end 70.4727 75.1473) (width 0.2) (layer "F.Cu") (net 7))
 (segment (start 69.905 86.4283) (end 70.3105 86.4283) (width 0.2) (layer "F.Cu") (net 7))
 (segment (start 70.4727 75.1473) (end 71.5 74.12) (width 0.2) (layer "F.Cu") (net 7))
 (segment (start 71.6015 85.1373) (end 71.6015 81.4139) (width 0.2) (layer "F.Cu") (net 7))
 (segment (start 69.905 87.58) (end 71.1817 87.58) (width 0.2) (layer "B.Cu") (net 7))
 (segment (start 73.88 83.93) (end 71.1817 86.6283) (width 0.2) (layer "B.Cu") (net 7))
 (segment (start 71.1817 86.6283) (end 71.1817 87.58) (width 0.2) (layer "B.Cu") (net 7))
 (segment (start 70.071 80.671) (end 71.1998 81.7998) (width 0.2) (layer "F.Cu") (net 6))
 (segment (start 69.905 85.08) (end 69.905 83.9283) (width 0.2) (layer "F.Cu") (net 6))
 (segment (start 71.5 71.04) (end 70.071 72.469) (width 0.2) (layer "F.Cu") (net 6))
 (segment (start 71.1998 83.0418) (end 70.3133 83.9283) (width 0.2) (layer "F.Cu") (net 6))
 (segment (start 70.3133 83.9283) (end 69.905 83.9283) (width 0.2) (layer "F.Cu") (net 6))
 (segment (start 71.1998 81.7998) (end 71.1998 83.0418) (width 0.2) (layer "F.Cu") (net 6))
 (segment (start 70.071 72.469) (end 70.071 80.671) (width 0.2) (layer "F.Cu") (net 6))
 (segment (start 71.1817 84.0883) (end 71.1817 85.08) (width 0.2) (layer "B.Cu") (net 6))
 (segment (start 73.88 81.39) (end 71.1817 84.0883) (width 0.2) (layer "B.Cu") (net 6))
 (segment (start 69.905 85.08) (end 71.1817 85.08) (width 0.2) (layer "B.Cu") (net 6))
 (segment (start 69 58.54) (end 69 59.6917) (width 0.2) (layer "F.Cu") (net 19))
 (segment (start 70.3498 62.6198) (end 70.3498 60.5898) (width 0.2) (layer "F.Cu") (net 19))
 (segment (start 73.88 66.15) (end 70.3498 62.6198) (width 0.2) (layer "F.Cu") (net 19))
 (segment (start 69.4517 59.6917) (end 69 59.6917) (width 0.2) (layer "F.Cu") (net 19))
 (segment (start 70.3498 60.5898) (end 69.4517 59.6917) (width 0.2) (layer "F.Cu") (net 19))
 (segment (start 72.4617 62.1917) (end 69 62.1917) (width 0.2) (layer "B.Cu") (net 18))
 (segment (start 69 61.04) (end 69 62.1917) (width 0.2) (layer "B.Cu") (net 18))
 (segment (start 73.88 63.61) (end 72.4617 62.1917) (width 0.2) (layer "B.Cu") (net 18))
 (segment (start 97.025 72.04) (end 97 72.015) (width 0.2) (layer "F.Cu") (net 8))
 (segment (start 97 72.015) (end 97 69.5) (width 0.2) (layer "F.Cu") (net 8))
 (segment (start 96.54 64.54) (end 96.54 55) (width 0.2) (layer "F.Cu") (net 2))
 (segment (start 97 65) (end 96.54 64.54) (width 0.2) (layer "F.Cu") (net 2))
 (segment (start 97 94.725) (end 97 90) (width 0.2) (layer "F.Cu") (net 9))
 (segment (start 97.025 94.75) (end 97 94.725) (width 0.2) (layer "F.Cu") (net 9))
 (segment (start 93 79) (end 90.6514 81.3486) (width 0.2) (layer "F.Cu") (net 3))
 (segment (start 90.6514 81.3486) (end 90.6514 100.1786) (width 0.2) (layer "F.Cu") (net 3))
 (segment (start 90.6514 100.1786) (end 89.12 101.71) (width 0.2) (layer "F.Cu") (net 3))
 (segment (start 92.3229 103.0671) (end 92.3229 92.6771) (width 0.2) (layer "F.Cu") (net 10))
 (segment (start 92.3229 92.6771) (end 95 90) (width 0.2) (layer "F.Cu") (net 10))
 (via (at 92.3229 103.0671) (size 0.6) (drill 0.3) (layers "F.Cu" "B.Cu") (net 10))
 (segment (start 73.88 101.71) (end 75.2371 103.0671) (width 0.2) (layer "B.Cu") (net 10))
 (segment (start 75.2371 103.0671) (end 92.3229 103.0671) (width 0.2) (layer "B.Cu") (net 10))
 (segment (start 94 48.17) (end 94 55) (width 0.2) (layer "F.Cu") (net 1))
 (segment (start 89.12 43.29) (end 94 48.17) (width 0.2) (layer "F.Cu") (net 1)))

